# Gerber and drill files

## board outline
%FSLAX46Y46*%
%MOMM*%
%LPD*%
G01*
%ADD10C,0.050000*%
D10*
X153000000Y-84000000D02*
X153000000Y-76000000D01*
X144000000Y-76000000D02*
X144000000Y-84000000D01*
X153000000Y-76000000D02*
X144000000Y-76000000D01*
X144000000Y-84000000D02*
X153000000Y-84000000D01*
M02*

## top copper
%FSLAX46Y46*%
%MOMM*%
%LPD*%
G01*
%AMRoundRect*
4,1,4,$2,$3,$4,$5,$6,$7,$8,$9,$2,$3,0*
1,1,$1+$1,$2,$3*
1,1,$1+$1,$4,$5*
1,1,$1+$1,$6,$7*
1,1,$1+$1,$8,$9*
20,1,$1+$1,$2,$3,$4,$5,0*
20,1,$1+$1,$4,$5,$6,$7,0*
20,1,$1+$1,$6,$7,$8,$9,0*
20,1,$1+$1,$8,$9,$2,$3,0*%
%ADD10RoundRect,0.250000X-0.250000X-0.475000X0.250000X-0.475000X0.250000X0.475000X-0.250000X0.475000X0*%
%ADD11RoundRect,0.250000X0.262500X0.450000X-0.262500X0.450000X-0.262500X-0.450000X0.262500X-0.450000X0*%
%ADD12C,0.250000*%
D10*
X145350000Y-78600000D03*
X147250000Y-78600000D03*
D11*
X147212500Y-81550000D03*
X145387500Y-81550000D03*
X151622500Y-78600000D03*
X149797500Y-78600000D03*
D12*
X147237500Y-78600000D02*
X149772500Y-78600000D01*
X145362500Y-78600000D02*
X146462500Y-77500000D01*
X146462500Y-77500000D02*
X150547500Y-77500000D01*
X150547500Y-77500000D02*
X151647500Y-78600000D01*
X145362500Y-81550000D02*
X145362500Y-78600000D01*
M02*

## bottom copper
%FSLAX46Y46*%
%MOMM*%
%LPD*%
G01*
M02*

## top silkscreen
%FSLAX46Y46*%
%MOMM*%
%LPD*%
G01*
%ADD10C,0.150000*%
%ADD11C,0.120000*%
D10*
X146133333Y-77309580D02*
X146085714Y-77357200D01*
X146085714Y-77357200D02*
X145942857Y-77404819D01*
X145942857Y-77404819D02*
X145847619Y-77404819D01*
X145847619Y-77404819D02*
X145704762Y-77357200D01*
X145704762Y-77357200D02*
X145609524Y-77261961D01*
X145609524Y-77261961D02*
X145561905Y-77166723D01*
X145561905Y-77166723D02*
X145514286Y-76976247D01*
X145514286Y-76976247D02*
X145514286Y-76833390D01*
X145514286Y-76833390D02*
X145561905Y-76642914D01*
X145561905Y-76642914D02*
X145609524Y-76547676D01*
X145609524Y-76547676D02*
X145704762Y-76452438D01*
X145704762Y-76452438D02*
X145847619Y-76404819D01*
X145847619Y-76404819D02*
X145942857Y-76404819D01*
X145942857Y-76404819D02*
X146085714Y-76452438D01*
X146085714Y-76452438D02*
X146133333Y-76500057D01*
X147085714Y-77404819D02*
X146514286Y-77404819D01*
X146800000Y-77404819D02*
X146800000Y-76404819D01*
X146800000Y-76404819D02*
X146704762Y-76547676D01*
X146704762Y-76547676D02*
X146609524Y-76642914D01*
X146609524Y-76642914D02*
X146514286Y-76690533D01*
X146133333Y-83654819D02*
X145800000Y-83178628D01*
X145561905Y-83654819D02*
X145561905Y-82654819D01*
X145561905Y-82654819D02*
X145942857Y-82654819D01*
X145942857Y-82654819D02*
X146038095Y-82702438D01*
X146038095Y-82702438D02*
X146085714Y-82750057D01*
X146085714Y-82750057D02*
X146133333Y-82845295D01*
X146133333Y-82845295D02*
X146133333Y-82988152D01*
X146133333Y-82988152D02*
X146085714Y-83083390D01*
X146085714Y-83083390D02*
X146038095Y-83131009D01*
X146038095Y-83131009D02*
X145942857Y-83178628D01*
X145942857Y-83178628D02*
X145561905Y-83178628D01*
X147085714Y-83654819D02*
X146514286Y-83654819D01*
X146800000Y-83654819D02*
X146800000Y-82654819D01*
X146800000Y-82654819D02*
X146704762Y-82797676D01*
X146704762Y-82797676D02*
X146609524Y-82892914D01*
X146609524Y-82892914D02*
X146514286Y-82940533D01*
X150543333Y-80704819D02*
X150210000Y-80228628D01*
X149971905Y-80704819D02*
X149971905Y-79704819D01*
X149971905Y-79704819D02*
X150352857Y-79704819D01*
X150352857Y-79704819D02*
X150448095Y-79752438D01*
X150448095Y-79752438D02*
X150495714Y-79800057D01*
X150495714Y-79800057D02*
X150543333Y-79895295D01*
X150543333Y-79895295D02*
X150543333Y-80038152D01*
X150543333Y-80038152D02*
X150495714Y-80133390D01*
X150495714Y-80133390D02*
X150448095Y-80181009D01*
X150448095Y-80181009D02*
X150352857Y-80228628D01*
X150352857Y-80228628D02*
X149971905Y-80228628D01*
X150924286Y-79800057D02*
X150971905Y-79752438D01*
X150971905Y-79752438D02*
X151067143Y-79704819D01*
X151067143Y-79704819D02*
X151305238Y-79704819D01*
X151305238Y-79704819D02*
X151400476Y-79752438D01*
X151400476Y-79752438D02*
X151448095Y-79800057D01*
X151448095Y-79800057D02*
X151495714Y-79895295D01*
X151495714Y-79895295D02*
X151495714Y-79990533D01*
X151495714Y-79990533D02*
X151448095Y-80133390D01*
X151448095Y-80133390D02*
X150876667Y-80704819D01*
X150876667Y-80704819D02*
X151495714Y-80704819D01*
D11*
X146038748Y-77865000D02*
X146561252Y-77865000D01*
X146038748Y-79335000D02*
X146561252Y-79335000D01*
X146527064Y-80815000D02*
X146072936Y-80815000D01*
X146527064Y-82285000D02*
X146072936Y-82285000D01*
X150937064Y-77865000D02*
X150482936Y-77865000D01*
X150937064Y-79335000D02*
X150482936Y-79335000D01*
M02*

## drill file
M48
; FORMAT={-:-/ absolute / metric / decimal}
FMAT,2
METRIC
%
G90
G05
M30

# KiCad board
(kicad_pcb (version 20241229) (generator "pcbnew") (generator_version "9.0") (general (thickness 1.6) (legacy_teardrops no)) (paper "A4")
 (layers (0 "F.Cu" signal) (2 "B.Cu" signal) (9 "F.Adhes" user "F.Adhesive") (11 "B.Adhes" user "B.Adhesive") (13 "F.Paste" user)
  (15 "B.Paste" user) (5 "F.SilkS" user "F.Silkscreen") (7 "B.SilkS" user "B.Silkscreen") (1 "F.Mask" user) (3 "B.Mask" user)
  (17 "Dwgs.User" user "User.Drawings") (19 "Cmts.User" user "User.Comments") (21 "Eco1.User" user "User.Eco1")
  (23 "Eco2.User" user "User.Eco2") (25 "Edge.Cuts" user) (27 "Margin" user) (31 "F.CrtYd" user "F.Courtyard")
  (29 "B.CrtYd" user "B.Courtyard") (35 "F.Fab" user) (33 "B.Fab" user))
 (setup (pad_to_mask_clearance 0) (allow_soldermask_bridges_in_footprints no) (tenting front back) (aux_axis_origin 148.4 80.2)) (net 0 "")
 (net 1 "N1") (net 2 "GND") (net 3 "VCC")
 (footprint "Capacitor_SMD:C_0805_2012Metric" (layer "F.Cu") (at 146.3 78.6)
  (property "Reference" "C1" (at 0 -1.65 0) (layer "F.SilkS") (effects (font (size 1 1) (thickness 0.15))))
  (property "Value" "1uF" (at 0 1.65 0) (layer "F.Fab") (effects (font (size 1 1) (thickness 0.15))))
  (fp_line (start -0.261252 -0.735) (end 0.261252 -0.735) (stroke (width 0.12) (type solid)) (layer "F.SilkS"))
  (fp_line (start -0.261252 0.735) (end 0.261252 0.735) (stroke (width 0.12) (type solid)) (layer "F.SilkS"))
  (pad "1" smd roundrect (at -0.95 0) (size 1 1.45) (layers "F.Cu" "F.Mask" "F.Paste") (roundrect_rratio 0.25) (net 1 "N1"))
  (pad "2" smd roundrect (at 0.95 0) (size 1 1.45) (layers "F.Cu" "F.Mask" "F.Paste") (roundrect_rratio 0.25) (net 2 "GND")))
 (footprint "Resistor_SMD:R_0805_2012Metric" (layer "F.Cu") (at 146.3 81.55 180)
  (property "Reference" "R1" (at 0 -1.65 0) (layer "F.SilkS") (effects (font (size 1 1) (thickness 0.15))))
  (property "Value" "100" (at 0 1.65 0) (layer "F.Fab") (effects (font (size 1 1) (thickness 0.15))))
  (fp_line (start -0.227064 0.735) (end 0.227064 0.735) (stroke (width 0.12) (type solid)) (layer "F.SilkS"))
  (fp_line (start -0.227064 -0.735) (end 0.227064 -0.735) (stroke (width 0.12) (type solid)) (layer "F.SilkS"))
  (pad "1" smd roundrect (at -0.9125 0 180) (size 1.025 1.4) (layers "F.Cu" "F.Mask" "F.Paste") (roundrect_rratio 0.243902) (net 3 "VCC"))
  (pad "2" smd roundrect (at 0.9125 0 180) (size 1.025 1.4) (layers "F.Cu" "F.Mask" "F.Paste") (roundrect_rratio 0.243902) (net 1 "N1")))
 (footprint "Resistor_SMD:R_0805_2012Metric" (layer "F.Cu") (at 150.71 78.6 180)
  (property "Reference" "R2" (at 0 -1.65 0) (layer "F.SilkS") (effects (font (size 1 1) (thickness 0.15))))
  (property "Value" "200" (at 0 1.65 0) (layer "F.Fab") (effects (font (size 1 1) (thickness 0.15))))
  (fp_line (start -0.227064 0.735) (end 0.227064 0.735) (stroke (width 0.12) (type solid)) (layer "F.SilkS"))
  (fp_line (start -0.227064 -0.735) (end 0.227064 -0.735) (stroke (width 0.12) (type solid)) (layer "F.SilkS"))
  (pad "1" smd roundrect (at -0.9125 0 180) (size 1.025 1.4) (layers "F.Cu" "F.Mask" "F.Paste") (roundrect_rratio 0.243902) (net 1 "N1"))
  (pad "2" smd roundrect (at 0.9125 0 180) (size 1.025 1.4) (layers "F.Cu" "F.Mask" "F.Paste") (roundrect_rratio 0.243902) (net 2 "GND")))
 (gr_line (start 153 84) (end 153 76) (stroke (width 0.05) (type solid)) (layer "Edge.Cuts"))
 (gr_line (start 144 76) (end 144 84) (stroke (width 0.05) (type solid)) (layer "Edge.Cuts"))
 (gr_line (start 153 76) (end 144 76) (stroke (width 0.05) (type solid)) (layer "Edge.Cuts"))
 (gr_line (start 144 84) (end 153 84) (stroke (width 0.05) (type solid)) (layer "Edge.Cuts"))
 (segment (start 147.2375 78.6) (end 149.7725 78.6) (width 0.25) (layer "F.Cu") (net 2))
 (segment (start 145.3625 78.6) (end 146.4625 77.5) (width 0.25) (layer "F.Cu") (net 1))
 (segment (start 146.4625 77.5) (end 150.5475 77.5) (width 0.25) (layer "F.Cu") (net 1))
 (segment (start 150.5475 77.5) (end 151.6475 78.6) (width 0.25) (layer "F.Cu") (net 1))
 (segment (start 145.3625 81.55) (end 145.3625 78.6) (width 0.25) (layer "F.Cu") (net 1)))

